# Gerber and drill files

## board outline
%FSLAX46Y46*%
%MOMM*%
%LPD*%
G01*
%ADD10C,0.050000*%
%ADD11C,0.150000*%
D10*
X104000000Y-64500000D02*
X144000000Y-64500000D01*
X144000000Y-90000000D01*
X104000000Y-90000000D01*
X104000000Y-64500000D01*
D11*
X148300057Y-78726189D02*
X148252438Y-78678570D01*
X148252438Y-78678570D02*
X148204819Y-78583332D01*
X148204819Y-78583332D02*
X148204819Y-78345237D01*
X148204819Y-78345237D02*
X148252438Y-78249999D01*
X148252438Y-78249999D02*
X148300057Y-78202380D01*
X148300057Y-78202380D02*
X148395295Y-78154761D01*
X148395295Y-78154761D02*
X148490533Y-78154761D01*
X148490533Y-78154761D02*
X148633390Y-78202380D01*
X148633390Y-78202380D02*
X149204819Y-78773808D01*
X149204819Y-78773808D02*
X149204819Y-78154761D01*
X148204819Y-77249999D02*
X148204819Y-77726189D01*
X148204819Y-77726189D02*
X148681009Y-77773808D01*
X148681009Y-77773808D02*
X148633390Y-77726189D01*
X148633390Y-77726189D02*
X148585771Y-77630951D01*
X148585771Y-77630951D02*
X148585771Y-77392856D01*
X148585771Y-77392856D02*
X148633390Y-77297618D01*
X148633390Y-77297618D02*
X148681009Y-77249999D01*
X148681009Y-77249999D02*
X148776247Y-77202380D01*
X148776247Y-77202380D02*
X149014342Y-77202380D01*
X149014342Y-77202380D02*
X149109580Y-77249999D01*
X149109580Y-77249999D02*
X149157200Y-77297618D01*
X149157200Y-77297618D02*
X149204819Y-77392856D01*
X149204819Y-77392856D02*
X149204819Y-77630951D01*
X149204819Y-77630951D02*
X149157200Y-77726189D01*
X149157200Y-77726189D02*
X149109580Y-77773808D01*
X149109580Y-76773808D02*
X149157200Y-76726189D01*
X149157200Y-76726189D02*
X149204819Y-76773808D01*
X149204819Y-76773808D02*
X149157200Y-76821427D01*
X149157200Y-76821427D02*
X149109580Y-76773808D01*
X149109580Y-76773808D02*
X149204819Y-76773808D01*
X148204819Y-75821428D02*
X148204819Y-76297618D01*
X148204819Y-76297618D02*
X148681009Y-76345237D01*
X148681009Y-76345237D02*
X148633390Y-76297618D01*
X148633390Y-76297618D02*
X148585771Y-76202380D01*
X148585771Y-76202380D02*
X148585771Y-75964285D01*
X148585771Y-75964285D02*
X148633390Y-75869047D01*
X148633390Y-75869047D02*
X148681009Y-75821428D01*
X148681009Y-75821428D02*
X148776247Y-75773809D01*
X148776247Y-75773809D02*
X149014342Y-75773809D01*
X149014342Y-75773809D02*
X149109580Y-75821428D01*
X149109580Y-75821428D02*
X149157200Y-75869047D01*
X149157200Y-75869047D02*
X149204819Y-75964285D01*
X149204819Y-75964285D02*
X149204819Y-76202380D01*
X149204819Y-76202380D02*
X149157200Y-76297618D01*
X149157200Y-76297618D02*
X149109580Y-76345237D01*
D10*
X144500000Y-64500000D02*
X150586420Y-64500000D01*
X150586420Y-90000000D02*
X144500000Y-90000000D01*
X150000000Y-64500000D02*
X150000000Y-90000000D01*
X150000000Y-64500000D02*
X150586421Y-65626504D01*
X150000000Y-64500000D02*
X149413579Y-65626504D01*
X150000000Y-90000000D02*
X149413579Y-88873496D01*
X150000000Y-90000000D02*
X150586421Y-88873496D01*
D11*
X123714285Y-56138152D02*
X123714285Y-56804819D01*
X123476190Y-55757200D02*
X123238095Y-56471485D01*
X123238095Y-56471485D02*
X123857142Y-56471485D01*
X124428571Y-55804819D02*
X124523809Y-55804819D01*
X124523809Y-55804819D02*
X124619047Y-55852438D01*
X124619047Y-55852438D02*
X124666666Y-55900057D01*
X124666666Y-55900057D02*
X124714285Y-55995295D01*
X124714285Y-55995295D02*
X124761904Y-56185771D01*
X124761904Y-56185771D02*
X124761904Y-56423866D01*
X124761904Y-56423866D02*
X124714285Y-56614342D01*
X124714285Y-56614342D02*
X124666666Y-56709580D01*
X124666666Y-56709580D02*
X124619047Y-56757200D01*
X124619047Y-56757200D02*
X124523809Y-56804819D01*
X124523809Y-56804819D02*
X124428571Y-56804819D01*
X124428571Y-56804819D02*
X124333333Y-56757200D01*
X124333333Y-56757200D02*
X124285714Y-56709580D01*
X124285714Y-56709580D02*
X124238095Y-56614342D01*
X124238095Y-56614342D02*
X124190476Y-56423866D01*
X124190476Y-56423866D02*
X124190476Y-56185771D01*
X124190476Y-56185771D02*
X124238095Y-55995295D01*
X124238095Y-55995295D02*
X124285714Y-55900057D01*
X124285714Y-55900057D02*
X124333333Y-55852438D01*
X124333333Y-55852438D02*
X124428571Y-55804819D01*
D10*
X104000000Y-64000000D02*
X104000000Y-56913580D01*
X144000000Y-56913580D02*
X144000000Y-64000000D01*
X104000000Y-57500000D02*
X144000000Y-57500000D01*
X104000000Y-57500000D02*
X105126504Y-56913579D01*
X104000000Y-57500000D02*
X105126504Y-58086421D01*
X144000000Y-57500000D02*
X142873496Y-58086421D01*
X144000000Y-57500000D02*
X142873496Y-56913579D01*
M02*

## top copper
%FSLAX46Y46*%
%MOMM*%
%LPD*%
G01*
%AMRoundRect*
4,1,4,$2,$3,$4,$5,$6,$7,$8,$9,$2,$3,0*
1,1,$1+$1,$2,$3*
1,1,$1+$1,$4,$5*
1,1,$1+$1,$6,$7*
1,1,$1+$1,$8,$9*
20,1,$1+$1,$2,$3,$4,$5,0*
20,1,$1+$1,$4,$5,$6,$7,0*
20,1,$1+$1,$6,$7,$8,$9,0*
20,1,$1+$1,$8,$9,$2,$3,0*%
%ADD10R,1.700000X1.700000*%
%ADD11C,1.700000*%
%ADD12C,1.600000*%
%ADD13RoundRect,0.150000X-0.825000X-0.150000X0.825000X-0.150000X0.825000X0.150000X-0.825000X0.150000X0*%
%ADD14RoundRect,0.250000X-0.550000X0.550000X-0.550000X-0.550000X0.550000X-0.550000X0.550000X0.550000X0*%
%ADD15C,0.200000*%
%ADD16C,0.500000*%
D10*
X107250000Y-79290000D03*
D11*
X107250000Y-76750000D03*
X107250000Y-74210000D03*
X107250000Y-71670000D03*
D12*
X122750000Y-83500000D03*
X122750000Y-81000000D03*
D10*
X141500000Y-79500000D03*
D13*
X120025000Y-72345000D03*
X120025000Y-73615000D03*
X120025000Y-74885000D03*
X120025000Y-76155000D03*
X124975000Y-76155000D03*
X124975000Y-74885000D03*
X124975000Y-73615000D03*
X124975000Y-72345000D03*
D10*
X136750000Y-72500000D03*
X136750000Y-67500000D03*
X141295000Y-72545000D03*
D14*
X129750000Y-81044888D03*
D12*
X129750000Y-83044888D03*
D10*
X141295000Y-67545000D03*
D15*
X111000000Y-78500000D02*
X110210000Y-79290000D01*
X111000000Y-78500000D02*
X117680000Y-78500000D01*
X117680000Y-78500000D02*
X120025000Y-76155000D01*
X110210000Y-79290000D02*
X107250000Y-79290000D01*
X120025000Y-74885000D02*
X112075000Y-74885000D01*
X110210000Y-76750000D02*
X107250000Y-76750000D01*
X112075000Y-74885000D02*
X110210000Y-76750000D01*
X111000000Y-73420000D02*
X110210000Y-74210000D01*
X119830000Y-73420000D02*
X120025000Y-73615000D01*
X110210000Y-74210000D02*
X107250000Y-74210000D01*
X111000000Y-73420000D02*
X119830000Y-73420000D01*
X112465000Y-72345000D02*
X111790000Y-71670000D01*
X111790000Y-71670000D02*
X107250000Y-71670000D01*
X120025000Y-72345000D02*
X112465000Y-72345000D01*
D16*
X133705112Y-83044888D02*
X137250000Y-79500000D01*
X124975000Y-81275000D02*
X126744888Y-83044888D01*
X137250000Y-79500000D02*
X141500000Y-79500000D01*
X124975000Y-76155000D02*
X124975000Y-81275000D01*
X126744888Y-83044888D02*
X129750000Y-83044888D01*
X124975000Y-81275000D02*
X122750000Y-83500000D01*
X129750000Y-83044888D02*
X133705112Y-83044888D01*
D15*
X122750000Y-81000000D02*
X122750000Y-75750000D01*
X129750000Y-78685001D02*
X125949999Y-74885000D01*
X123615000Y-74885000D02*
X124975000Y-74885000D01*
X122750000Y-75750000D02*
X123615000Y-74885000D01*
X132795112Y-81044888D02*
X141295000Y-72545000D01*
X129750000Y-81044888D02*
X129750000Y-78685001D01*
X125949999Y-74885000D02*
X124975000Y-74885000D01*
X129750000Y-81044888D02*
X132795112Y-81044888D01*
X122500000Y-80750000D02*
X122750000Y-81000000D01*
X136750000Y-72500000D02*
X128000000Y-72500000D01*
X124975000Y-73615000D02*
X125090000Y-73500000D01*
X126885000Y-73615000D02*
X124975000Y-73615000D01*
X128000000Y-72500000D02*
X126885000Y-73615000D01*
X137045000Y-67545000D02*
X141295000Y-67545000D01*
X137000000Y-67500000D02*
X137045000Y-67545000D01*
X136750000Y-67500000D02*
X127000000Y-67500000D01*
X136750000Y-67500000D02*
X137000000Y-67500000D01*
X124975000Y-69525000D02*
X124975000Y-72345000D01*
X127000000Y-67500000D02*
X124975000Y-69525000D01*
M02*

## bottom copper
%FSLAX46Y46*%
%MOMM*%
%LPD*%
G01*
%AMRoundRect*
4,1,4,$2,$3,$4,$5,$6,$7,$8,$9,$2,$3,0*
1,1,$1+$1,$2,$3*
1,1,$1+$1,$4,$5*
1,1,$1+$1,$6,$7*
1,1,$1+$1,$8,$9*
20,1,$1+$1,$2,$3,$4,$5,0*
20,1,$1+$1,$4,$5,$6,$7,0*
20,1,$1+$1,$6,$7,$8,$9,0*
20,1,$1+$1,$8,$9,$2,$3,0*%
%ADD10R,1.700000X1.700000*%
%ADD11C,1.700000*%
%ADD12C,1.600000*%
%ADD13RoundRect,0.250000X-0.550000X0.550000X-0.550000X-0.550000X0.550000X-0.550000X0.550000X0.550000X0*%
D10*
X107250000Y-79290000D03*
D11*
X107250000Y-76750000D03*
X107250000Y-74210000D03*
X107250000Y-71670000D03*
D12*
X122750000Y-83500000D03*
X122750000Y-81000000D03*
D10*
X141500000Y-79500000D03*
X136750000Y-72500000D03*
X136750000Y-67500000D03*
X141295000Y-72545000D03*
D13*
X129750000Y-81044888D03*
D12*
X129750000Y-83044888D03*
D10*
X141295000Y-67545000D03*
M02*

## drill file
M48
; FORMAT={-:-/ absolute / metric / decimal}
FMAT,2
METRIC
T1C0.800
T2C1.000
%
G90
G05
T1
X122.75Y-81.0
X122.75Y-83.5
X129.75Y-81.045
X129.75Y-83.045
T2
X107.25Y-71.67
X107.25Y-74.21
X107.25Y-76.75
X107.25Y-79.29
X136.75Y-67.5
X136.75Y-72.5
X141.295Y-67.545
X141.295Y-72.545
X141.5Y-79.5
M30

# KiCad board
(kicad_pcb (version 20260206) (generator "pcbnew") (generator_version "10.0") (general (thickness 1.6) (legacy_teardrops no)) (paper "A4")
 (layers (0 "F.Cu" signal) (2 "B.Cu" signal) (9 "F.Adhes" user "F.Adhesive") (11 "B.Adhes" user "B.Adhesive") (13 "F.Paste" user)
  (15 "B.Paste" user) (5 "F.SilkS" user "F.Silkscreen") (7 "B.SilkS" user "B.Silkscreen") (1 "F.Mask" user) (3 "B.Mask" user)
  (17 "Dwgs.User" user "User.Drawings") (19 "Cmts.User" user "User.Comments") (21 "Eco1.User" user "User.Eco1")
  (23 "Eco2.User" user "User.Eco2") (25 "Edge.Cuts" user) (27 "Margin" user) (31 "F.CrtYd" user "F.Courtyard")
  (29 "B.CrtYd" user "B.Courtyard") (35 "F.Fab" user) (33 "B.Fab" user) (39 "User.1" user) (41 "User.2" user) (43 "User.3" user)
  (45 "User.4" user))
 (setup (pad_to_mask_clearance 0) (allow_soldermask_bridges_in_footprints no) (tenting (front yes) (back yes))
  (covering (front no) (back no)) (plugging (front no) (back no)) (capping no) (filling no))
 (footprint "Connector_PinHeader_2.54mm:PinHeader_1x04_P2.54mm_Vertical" (layer "F.Cu") (at 107.25 79.29 180)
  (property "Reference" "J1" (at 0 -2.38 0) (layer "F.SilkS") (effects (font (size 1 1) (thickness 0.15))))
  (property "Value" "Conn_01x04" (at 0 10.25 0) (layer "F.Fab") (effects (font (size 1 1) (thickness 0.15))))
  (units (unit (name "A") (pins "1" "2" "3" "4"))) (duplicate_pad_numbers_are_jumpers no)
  (pad "1" thru_hole rect (at 0 0 180) (size 1.7 1.7) (drill 1) (layers "*.Cu" "*.Mask") (remove_unused_layers no) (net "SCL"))
  (pad "2" thru_hole circle (at 0 2.54 180) (size 1.7 1.7) (drill 1) (layers "*.Cu" "*.Mask") (remove_unused_layers no) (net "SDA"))
  (pad "3" thru_hole circle (at 0 5.08 180) (size 1.7 1.7) (drill 1) (layers "*.Cu" "*.Mask") (remove_unused_layers no) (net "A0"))
  (pad "4" thru_hole circle (at 0 7.62 180) (size 1.7 1.7) (drill 1) (layers "*.Cu" "*.Mask") (remove_unused_layers no) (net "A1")))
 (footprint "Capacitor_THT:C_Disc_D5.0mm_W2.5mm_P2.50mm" (layer "F.Cu") (at 122.75 83.5 90)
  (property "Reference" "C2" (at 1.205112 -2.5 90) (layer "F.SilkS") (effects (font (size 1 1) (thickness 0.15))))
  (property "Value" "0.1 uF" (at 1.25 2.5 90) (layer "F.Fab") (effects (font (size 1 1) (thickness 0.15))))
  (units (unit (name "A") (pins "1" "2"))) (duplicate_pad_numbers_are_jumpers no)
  (pad "1" thru_hole circle (at 0 0 90) (size 1.6 1.6) (drill 0.8) (layers "*.Cu" "*.Mask") (remove_unused_layers no) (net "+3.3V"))
  (pad "2" thru_hole circle (at 2.5 0 90) (size 1.6 1.6) (drill 0.8) (layers "*.Cu" "*.Mask") (remove_unused_layers no) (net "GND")))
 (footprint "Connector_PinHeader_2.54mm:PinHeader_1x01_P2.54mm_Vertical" (layer "F.Cu") (at 141.5 79.5)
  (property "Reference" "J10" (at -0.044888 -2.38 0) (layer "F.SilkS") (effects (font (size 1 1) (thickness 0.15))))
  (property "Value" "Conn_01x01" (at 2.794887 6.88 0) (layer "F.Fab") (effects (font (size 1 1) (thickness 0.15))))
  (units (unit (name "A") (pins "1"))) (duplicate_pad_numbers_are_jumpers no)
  (pad "1" thru_hole rect (at 0 0) (size 1.7 1.7) (drill 1) (layers "*.Cu" "*.Mask") (remove_unused_layers no) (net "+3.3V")))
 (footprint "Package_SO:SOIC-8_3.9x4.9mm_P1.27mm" (layer "F.Cu") (at 122.5 74.25)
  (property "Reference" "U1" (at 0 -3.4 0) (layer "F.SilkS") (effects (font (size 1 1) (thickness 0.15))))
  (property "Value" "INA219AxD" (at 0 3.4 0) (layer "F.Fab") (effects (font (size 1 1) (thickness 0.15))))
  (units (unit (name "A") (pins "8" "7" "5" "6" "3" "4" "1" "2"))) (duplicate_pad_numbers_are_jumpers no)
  (pad "1" smd roundrect (at -2.475 -1.905) (size 1.95 0.6) (layers "F.Cu" "F.Mask" "F.Paste") (roundrect_rratio 0.25) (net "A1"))
  (pad "2" smd roundrect (at -2.475 -0.635) (size 1.95 0.6) (layers "F.Cu" "F.Mask" "F.Paste") (roundrect_rratio 0.25) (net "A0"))
  (pad "3" smd roundrect (at -2.475 0.635) (size 1.95 0.6) (layers "F.Cu" "F.Mask" "F.Paste") (roundrect_rratio 0.25) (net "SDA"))
  (pad "4" smd roundrect (at -2.475 1.905) (size 1.95 0.6) (layers "F.Cu" "F.Mask" "F.Paste") (roundrect_rratio 0.25) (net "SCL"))
  (pad "5" smd roundrect (at 2.475 1.905) (size 1.95 0.6) (layers "F.Cu" "F.Mask" "F.Paste") (roundrect_rratio 0.25) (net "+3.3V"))
  (pad "6" smd roundrect (at 2.475 0.635) (size 1.95 0.6) (layers "F.Cu" "F.Mask" "F.Paste") (roundrect_rratio 0.25) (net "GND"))
  (pad "7" smd roundrect (at 2.475 -0.635) (size 1.95 0.6) (layers "F.Cu" "F.Mask" "F.Paste") (roundrect_rratio 0.25)
   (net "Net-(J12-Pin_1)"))
  (pad "8" smd roundrect (at 2.475 -1.905) (size 1.95 0.6) (layers "F.Cu" "F.Mask" "F.Paste") (roundrect_rratio 0.25)
   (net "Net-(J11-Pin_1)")))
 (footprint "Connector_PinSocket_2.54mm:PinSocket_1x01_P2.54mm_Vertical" (layer "F.Cu") (at 136.75 72.5)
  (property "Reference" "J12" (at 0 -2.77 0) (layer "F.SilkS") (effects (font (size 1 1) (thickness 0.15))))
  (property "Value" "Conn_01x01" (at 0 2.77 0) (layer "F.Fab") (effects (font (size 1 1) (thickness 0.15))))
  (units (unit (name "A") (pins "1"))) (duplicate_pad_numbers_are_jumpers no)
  (pad "1" thru_hole rect (at 0 0) (size 1.7 1.7) (drill 1) (layers "*.Cu" "*.Mask") (remove_unused_layers no) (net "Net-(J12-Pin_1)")))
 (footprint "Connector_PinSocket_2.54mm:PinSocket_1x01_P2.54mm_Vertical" (layer "F.Cu") (at 136.75 67.5)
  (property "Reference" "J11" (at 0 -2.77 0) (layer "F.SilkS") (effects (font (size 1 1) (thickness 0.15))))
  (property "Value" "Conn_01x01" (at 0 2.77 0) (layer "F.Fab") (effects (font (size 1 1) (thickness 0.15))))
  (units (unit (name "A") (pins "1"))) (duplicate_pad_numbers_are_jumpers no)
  (pad "1" thru_hole rect (at 0 0) (size 1.7 1.7) (drill 1) (layers "*.Cu" "*.Mask") (remove_unused_layers no) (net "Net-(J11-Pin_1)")))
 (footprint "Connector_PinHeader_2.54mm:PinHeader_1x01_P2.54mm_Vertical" (layer "F.Cu") (at 141.295 72.545)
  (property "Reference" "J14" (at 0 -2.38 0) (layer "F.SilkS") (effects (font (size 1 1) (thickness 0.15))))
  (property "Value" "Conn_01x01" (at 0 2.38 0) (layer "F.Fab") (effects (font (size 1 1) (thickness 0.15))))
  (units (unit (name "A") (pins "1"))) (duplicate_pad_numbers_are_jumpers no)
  (pad "1" thru_hole rect (at 0 0) (size 1.7 1.7) (drill 1) (layers "*.Cu" "*.Mask") (remove_unused_layers no) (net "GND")))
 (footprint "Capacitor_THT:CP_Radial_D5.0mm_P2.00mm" (layer "F.Cu") (at 129.75 81.044888 -90)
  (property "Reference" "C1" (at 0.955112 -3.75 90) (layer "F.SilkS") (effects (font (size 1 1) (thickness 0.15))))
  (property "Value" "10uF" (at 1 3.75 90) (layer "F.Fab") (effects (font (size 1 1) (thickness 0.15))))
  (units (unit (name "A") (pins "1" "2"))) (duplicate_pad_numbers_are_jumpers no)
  (pad "1" thru_hole roundrect (at 0 0 270) (size 1.6 1.6) (drill 0.8) (layers "*.Cu" "*.Mask") (remove_unused_layers no)
   (roundrect_rratio 0.15625) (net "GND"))
  (pad "2" thru_hole circle (at 2 0 270) (size 1.6 1.6) (drill 0.8) (layers "*.Cu" "*.Mask") (remove_unused_layers no) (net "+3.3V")))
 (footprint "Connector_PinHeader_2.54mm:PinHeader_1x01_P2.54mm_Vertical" (layer "F.Cu") (at 141.295 67.545)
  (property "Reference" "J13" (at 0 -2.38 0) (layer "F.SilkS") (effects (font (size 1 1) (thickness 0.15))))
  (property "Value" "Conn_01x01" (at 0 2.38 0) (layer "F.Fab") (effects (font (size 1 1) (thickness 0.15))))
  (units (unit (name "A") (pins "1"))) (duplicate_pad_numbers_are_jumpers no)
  (pad "1" thru_hole rect (at 0 0) (size 1.7 1.7) (drill 1) (layers "*.Cu" "*.Mask") (remove_unused_layers no) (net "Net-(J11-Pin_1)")))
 (gr_rect (start 104 64.5) (end 144 90) (stroke (width 0.05) (type default)) (fill no) (layer "Edge.Cuts"))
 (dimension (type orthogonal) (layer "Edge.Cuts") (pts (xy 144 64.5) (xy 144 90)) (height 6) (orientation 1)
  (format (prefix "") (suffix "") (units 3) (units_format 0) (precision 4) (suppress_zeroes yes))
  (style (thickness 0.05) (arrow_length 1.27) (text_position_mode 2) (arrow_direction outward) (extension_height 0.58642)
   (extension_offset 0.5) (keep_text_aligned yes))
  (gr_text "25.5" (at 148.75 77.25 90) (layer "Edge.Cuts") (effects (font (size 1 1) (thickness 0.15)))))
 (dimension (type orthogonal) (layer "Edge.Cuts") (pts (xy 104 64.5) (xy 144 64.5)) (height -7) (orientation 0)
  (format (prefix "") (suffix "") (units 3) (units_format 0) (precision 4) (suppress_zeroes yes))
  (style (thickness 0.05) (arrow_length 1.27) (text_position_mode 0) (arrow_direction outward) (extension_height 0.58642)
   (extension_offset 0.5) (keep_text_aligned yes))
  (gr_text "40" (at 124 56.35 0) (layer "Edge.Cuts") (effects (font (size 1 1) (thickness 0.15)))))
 (segment (start 111 78.5) (end 110.21 79.29) (width 0.2) (layer "F.Cu") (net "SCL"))
 (segment (start 111 78.5) (end 117.68 78.5) (width 0.2) (layer "F.Cu") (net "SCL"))
 (segment (start 117.68 78.5) (end 120.025 76.155) (width 0.2) (layer "F.Cu") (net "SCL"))
 (segment (start 110.21 79.29) (end 107.25 79.29) (width 0.2) (layer "F.Cu") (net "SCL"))
 (segment (start 120.025 74.885) (end 112.075 74.885) (width 0.2) (layer "F.Cu") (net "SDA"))
 (segment (start 110.21 76.75) (end 107.25 76.75) (width 0.2) (layer "F.Cu") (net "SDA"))
 (segment (start 112.075 74.885) (end 110.21 76.75) (width 0.2) (layer "F.Cu") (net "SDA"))
 (segment (start 111 73.42) (end 110.21 74.21) (width 0.2) (layer "F.Cu") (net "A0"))
 (segment (start 119.83 73.42) (end 120.025 73.615) (width 0.2) (layer "F.Cu") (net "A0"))
 (segment (start 110.21 74.21) (end 107.25 74.21) (width 0.2) (layer "F.Cu") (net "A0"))
 (segment (start 111 73.42) (end 119.83 73.42) (width 0.2) (layer "F.Cu") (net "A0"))
 (segment (start 112.465 72.345) (end 111.79 71.67) (width 0.2) (layer "F.Cu") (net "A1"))
 (segment (start 111.79 71.67) (end 107.25 71.67) (width 0.2) (layer "F.Cu") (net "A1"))
 (segment (start 120.025 72.345) (end 112.465 72.345) (width 0.2) (layer "F.Cu") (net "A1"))
 (segment (start 133.705112 83.044888) (end 137.25 79.5) (width 0.5) (layer "F.Cu") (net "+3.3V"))
 (segment (start 124.975 81.275) (end 126.744888 83.044888) (width 0.5) (layer "F.Cu") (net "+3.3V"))
 (segment (start 137.25 79.5) (end 141.5 79.5) (width 0.5) (layer "F.Cu") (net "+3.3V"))
 (segment (start 124.975 76.155) (end 124.975 81.275) (width 0.5) (layer "F.Cu") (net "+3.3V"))
 (segment (start 126.744888 83.044888) (end 129.75 83.044888) (width 0.5) (layer "F.Cu") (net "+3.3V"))
 (segment (start 124.975 81.275) (end 122.75 83.5) (width 0.5) (layer "F.Cu") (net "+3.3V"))
 (segment (start 129.75 83.044888) (end 133.705112 83.044888) (width 0.5) (layer "F.Cu") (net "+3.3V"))
 (segment (start 122.75 81) (end 122.75 75.75) (width 0.2) (layer "F.Cu") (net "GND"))
 (segment (start 129.75 78.685001) (end 125.949999 74.885) (width 0.2) (layer "F.Cu") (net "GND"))
 (segment (start 123.615 74.885) (end 124.975 74.885) (width 0.2) (layer "F.Cu") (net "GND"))
 (segment (start 122.75 75.75) (end 123.615 74.885) (width 0.2) (layer "F.Cu") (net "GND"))
 (segment (start 132.795112 81.044888) (end 141.295 72.545) (width 0.2) (layer "F.Cu") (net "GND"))
 (segment (start 129.75 81.044888) (end 129.75 78.685001) (width 0.2) (layer "F.Cu") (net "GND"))
 (segment (start 125.949999 74.885) (end 124.975 74.885) (width 0.2) (layer "F.Cu") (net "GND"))
 (segment (start 129.75 81.044888) (end 132.795112 81.044888) (width 0.2) (layer "F.Cu") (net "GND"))
 (segment (start 122.5 80.75) (end 122.75 81) (width 0.2) (layer "F.Cu") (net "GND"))
 (segment (start 136.75 72.5) (end 128 72.5) (width 0.2) (layer "F.Cu") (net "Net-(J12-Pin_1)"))
 (segment (start 124.975 73.615) (end 125.09 73.5) (width 0.2) (layer "F.Cu") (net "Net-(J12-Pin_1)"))
 (segment (start 126.885 73.615) (end 124.975 73.615) (width 0.2) (layer "F.Cu") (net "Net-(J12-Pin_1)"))
 (segment (start 128 72.5) (end 126.885 73.615) (width 0.2) (layer "F.Cu") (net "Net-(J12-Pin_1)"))
 (segment (start 137.045 67.545) (end 141.295 67.545) (width 0.2) (layer "F.Cu") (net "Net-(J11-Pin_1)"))
 (segment (start 137 67.5) (end 137.045 67.545) (width 0.2) (layer "F.Cu") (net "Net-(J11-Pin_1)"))
 (segment (start 136.75 67.5) (end 127 67.5) (width 0.2) (layer "F.Cu") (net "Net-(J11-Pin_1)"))
 (segment (start 136.75 67.5) (end 137 67.5) (width 0.2) (layer "F.Cu") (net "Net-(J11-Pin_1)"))
 (segment (start 124.975 69.525) (end 124.975 72.345) (width 0.2) (layer "F.Cu") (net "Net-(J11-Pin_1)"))
 (segment (start 127 67.5) (end 124.975 69.525) (width 0.2) (layer "F.Cu") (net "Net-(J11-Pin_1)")))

